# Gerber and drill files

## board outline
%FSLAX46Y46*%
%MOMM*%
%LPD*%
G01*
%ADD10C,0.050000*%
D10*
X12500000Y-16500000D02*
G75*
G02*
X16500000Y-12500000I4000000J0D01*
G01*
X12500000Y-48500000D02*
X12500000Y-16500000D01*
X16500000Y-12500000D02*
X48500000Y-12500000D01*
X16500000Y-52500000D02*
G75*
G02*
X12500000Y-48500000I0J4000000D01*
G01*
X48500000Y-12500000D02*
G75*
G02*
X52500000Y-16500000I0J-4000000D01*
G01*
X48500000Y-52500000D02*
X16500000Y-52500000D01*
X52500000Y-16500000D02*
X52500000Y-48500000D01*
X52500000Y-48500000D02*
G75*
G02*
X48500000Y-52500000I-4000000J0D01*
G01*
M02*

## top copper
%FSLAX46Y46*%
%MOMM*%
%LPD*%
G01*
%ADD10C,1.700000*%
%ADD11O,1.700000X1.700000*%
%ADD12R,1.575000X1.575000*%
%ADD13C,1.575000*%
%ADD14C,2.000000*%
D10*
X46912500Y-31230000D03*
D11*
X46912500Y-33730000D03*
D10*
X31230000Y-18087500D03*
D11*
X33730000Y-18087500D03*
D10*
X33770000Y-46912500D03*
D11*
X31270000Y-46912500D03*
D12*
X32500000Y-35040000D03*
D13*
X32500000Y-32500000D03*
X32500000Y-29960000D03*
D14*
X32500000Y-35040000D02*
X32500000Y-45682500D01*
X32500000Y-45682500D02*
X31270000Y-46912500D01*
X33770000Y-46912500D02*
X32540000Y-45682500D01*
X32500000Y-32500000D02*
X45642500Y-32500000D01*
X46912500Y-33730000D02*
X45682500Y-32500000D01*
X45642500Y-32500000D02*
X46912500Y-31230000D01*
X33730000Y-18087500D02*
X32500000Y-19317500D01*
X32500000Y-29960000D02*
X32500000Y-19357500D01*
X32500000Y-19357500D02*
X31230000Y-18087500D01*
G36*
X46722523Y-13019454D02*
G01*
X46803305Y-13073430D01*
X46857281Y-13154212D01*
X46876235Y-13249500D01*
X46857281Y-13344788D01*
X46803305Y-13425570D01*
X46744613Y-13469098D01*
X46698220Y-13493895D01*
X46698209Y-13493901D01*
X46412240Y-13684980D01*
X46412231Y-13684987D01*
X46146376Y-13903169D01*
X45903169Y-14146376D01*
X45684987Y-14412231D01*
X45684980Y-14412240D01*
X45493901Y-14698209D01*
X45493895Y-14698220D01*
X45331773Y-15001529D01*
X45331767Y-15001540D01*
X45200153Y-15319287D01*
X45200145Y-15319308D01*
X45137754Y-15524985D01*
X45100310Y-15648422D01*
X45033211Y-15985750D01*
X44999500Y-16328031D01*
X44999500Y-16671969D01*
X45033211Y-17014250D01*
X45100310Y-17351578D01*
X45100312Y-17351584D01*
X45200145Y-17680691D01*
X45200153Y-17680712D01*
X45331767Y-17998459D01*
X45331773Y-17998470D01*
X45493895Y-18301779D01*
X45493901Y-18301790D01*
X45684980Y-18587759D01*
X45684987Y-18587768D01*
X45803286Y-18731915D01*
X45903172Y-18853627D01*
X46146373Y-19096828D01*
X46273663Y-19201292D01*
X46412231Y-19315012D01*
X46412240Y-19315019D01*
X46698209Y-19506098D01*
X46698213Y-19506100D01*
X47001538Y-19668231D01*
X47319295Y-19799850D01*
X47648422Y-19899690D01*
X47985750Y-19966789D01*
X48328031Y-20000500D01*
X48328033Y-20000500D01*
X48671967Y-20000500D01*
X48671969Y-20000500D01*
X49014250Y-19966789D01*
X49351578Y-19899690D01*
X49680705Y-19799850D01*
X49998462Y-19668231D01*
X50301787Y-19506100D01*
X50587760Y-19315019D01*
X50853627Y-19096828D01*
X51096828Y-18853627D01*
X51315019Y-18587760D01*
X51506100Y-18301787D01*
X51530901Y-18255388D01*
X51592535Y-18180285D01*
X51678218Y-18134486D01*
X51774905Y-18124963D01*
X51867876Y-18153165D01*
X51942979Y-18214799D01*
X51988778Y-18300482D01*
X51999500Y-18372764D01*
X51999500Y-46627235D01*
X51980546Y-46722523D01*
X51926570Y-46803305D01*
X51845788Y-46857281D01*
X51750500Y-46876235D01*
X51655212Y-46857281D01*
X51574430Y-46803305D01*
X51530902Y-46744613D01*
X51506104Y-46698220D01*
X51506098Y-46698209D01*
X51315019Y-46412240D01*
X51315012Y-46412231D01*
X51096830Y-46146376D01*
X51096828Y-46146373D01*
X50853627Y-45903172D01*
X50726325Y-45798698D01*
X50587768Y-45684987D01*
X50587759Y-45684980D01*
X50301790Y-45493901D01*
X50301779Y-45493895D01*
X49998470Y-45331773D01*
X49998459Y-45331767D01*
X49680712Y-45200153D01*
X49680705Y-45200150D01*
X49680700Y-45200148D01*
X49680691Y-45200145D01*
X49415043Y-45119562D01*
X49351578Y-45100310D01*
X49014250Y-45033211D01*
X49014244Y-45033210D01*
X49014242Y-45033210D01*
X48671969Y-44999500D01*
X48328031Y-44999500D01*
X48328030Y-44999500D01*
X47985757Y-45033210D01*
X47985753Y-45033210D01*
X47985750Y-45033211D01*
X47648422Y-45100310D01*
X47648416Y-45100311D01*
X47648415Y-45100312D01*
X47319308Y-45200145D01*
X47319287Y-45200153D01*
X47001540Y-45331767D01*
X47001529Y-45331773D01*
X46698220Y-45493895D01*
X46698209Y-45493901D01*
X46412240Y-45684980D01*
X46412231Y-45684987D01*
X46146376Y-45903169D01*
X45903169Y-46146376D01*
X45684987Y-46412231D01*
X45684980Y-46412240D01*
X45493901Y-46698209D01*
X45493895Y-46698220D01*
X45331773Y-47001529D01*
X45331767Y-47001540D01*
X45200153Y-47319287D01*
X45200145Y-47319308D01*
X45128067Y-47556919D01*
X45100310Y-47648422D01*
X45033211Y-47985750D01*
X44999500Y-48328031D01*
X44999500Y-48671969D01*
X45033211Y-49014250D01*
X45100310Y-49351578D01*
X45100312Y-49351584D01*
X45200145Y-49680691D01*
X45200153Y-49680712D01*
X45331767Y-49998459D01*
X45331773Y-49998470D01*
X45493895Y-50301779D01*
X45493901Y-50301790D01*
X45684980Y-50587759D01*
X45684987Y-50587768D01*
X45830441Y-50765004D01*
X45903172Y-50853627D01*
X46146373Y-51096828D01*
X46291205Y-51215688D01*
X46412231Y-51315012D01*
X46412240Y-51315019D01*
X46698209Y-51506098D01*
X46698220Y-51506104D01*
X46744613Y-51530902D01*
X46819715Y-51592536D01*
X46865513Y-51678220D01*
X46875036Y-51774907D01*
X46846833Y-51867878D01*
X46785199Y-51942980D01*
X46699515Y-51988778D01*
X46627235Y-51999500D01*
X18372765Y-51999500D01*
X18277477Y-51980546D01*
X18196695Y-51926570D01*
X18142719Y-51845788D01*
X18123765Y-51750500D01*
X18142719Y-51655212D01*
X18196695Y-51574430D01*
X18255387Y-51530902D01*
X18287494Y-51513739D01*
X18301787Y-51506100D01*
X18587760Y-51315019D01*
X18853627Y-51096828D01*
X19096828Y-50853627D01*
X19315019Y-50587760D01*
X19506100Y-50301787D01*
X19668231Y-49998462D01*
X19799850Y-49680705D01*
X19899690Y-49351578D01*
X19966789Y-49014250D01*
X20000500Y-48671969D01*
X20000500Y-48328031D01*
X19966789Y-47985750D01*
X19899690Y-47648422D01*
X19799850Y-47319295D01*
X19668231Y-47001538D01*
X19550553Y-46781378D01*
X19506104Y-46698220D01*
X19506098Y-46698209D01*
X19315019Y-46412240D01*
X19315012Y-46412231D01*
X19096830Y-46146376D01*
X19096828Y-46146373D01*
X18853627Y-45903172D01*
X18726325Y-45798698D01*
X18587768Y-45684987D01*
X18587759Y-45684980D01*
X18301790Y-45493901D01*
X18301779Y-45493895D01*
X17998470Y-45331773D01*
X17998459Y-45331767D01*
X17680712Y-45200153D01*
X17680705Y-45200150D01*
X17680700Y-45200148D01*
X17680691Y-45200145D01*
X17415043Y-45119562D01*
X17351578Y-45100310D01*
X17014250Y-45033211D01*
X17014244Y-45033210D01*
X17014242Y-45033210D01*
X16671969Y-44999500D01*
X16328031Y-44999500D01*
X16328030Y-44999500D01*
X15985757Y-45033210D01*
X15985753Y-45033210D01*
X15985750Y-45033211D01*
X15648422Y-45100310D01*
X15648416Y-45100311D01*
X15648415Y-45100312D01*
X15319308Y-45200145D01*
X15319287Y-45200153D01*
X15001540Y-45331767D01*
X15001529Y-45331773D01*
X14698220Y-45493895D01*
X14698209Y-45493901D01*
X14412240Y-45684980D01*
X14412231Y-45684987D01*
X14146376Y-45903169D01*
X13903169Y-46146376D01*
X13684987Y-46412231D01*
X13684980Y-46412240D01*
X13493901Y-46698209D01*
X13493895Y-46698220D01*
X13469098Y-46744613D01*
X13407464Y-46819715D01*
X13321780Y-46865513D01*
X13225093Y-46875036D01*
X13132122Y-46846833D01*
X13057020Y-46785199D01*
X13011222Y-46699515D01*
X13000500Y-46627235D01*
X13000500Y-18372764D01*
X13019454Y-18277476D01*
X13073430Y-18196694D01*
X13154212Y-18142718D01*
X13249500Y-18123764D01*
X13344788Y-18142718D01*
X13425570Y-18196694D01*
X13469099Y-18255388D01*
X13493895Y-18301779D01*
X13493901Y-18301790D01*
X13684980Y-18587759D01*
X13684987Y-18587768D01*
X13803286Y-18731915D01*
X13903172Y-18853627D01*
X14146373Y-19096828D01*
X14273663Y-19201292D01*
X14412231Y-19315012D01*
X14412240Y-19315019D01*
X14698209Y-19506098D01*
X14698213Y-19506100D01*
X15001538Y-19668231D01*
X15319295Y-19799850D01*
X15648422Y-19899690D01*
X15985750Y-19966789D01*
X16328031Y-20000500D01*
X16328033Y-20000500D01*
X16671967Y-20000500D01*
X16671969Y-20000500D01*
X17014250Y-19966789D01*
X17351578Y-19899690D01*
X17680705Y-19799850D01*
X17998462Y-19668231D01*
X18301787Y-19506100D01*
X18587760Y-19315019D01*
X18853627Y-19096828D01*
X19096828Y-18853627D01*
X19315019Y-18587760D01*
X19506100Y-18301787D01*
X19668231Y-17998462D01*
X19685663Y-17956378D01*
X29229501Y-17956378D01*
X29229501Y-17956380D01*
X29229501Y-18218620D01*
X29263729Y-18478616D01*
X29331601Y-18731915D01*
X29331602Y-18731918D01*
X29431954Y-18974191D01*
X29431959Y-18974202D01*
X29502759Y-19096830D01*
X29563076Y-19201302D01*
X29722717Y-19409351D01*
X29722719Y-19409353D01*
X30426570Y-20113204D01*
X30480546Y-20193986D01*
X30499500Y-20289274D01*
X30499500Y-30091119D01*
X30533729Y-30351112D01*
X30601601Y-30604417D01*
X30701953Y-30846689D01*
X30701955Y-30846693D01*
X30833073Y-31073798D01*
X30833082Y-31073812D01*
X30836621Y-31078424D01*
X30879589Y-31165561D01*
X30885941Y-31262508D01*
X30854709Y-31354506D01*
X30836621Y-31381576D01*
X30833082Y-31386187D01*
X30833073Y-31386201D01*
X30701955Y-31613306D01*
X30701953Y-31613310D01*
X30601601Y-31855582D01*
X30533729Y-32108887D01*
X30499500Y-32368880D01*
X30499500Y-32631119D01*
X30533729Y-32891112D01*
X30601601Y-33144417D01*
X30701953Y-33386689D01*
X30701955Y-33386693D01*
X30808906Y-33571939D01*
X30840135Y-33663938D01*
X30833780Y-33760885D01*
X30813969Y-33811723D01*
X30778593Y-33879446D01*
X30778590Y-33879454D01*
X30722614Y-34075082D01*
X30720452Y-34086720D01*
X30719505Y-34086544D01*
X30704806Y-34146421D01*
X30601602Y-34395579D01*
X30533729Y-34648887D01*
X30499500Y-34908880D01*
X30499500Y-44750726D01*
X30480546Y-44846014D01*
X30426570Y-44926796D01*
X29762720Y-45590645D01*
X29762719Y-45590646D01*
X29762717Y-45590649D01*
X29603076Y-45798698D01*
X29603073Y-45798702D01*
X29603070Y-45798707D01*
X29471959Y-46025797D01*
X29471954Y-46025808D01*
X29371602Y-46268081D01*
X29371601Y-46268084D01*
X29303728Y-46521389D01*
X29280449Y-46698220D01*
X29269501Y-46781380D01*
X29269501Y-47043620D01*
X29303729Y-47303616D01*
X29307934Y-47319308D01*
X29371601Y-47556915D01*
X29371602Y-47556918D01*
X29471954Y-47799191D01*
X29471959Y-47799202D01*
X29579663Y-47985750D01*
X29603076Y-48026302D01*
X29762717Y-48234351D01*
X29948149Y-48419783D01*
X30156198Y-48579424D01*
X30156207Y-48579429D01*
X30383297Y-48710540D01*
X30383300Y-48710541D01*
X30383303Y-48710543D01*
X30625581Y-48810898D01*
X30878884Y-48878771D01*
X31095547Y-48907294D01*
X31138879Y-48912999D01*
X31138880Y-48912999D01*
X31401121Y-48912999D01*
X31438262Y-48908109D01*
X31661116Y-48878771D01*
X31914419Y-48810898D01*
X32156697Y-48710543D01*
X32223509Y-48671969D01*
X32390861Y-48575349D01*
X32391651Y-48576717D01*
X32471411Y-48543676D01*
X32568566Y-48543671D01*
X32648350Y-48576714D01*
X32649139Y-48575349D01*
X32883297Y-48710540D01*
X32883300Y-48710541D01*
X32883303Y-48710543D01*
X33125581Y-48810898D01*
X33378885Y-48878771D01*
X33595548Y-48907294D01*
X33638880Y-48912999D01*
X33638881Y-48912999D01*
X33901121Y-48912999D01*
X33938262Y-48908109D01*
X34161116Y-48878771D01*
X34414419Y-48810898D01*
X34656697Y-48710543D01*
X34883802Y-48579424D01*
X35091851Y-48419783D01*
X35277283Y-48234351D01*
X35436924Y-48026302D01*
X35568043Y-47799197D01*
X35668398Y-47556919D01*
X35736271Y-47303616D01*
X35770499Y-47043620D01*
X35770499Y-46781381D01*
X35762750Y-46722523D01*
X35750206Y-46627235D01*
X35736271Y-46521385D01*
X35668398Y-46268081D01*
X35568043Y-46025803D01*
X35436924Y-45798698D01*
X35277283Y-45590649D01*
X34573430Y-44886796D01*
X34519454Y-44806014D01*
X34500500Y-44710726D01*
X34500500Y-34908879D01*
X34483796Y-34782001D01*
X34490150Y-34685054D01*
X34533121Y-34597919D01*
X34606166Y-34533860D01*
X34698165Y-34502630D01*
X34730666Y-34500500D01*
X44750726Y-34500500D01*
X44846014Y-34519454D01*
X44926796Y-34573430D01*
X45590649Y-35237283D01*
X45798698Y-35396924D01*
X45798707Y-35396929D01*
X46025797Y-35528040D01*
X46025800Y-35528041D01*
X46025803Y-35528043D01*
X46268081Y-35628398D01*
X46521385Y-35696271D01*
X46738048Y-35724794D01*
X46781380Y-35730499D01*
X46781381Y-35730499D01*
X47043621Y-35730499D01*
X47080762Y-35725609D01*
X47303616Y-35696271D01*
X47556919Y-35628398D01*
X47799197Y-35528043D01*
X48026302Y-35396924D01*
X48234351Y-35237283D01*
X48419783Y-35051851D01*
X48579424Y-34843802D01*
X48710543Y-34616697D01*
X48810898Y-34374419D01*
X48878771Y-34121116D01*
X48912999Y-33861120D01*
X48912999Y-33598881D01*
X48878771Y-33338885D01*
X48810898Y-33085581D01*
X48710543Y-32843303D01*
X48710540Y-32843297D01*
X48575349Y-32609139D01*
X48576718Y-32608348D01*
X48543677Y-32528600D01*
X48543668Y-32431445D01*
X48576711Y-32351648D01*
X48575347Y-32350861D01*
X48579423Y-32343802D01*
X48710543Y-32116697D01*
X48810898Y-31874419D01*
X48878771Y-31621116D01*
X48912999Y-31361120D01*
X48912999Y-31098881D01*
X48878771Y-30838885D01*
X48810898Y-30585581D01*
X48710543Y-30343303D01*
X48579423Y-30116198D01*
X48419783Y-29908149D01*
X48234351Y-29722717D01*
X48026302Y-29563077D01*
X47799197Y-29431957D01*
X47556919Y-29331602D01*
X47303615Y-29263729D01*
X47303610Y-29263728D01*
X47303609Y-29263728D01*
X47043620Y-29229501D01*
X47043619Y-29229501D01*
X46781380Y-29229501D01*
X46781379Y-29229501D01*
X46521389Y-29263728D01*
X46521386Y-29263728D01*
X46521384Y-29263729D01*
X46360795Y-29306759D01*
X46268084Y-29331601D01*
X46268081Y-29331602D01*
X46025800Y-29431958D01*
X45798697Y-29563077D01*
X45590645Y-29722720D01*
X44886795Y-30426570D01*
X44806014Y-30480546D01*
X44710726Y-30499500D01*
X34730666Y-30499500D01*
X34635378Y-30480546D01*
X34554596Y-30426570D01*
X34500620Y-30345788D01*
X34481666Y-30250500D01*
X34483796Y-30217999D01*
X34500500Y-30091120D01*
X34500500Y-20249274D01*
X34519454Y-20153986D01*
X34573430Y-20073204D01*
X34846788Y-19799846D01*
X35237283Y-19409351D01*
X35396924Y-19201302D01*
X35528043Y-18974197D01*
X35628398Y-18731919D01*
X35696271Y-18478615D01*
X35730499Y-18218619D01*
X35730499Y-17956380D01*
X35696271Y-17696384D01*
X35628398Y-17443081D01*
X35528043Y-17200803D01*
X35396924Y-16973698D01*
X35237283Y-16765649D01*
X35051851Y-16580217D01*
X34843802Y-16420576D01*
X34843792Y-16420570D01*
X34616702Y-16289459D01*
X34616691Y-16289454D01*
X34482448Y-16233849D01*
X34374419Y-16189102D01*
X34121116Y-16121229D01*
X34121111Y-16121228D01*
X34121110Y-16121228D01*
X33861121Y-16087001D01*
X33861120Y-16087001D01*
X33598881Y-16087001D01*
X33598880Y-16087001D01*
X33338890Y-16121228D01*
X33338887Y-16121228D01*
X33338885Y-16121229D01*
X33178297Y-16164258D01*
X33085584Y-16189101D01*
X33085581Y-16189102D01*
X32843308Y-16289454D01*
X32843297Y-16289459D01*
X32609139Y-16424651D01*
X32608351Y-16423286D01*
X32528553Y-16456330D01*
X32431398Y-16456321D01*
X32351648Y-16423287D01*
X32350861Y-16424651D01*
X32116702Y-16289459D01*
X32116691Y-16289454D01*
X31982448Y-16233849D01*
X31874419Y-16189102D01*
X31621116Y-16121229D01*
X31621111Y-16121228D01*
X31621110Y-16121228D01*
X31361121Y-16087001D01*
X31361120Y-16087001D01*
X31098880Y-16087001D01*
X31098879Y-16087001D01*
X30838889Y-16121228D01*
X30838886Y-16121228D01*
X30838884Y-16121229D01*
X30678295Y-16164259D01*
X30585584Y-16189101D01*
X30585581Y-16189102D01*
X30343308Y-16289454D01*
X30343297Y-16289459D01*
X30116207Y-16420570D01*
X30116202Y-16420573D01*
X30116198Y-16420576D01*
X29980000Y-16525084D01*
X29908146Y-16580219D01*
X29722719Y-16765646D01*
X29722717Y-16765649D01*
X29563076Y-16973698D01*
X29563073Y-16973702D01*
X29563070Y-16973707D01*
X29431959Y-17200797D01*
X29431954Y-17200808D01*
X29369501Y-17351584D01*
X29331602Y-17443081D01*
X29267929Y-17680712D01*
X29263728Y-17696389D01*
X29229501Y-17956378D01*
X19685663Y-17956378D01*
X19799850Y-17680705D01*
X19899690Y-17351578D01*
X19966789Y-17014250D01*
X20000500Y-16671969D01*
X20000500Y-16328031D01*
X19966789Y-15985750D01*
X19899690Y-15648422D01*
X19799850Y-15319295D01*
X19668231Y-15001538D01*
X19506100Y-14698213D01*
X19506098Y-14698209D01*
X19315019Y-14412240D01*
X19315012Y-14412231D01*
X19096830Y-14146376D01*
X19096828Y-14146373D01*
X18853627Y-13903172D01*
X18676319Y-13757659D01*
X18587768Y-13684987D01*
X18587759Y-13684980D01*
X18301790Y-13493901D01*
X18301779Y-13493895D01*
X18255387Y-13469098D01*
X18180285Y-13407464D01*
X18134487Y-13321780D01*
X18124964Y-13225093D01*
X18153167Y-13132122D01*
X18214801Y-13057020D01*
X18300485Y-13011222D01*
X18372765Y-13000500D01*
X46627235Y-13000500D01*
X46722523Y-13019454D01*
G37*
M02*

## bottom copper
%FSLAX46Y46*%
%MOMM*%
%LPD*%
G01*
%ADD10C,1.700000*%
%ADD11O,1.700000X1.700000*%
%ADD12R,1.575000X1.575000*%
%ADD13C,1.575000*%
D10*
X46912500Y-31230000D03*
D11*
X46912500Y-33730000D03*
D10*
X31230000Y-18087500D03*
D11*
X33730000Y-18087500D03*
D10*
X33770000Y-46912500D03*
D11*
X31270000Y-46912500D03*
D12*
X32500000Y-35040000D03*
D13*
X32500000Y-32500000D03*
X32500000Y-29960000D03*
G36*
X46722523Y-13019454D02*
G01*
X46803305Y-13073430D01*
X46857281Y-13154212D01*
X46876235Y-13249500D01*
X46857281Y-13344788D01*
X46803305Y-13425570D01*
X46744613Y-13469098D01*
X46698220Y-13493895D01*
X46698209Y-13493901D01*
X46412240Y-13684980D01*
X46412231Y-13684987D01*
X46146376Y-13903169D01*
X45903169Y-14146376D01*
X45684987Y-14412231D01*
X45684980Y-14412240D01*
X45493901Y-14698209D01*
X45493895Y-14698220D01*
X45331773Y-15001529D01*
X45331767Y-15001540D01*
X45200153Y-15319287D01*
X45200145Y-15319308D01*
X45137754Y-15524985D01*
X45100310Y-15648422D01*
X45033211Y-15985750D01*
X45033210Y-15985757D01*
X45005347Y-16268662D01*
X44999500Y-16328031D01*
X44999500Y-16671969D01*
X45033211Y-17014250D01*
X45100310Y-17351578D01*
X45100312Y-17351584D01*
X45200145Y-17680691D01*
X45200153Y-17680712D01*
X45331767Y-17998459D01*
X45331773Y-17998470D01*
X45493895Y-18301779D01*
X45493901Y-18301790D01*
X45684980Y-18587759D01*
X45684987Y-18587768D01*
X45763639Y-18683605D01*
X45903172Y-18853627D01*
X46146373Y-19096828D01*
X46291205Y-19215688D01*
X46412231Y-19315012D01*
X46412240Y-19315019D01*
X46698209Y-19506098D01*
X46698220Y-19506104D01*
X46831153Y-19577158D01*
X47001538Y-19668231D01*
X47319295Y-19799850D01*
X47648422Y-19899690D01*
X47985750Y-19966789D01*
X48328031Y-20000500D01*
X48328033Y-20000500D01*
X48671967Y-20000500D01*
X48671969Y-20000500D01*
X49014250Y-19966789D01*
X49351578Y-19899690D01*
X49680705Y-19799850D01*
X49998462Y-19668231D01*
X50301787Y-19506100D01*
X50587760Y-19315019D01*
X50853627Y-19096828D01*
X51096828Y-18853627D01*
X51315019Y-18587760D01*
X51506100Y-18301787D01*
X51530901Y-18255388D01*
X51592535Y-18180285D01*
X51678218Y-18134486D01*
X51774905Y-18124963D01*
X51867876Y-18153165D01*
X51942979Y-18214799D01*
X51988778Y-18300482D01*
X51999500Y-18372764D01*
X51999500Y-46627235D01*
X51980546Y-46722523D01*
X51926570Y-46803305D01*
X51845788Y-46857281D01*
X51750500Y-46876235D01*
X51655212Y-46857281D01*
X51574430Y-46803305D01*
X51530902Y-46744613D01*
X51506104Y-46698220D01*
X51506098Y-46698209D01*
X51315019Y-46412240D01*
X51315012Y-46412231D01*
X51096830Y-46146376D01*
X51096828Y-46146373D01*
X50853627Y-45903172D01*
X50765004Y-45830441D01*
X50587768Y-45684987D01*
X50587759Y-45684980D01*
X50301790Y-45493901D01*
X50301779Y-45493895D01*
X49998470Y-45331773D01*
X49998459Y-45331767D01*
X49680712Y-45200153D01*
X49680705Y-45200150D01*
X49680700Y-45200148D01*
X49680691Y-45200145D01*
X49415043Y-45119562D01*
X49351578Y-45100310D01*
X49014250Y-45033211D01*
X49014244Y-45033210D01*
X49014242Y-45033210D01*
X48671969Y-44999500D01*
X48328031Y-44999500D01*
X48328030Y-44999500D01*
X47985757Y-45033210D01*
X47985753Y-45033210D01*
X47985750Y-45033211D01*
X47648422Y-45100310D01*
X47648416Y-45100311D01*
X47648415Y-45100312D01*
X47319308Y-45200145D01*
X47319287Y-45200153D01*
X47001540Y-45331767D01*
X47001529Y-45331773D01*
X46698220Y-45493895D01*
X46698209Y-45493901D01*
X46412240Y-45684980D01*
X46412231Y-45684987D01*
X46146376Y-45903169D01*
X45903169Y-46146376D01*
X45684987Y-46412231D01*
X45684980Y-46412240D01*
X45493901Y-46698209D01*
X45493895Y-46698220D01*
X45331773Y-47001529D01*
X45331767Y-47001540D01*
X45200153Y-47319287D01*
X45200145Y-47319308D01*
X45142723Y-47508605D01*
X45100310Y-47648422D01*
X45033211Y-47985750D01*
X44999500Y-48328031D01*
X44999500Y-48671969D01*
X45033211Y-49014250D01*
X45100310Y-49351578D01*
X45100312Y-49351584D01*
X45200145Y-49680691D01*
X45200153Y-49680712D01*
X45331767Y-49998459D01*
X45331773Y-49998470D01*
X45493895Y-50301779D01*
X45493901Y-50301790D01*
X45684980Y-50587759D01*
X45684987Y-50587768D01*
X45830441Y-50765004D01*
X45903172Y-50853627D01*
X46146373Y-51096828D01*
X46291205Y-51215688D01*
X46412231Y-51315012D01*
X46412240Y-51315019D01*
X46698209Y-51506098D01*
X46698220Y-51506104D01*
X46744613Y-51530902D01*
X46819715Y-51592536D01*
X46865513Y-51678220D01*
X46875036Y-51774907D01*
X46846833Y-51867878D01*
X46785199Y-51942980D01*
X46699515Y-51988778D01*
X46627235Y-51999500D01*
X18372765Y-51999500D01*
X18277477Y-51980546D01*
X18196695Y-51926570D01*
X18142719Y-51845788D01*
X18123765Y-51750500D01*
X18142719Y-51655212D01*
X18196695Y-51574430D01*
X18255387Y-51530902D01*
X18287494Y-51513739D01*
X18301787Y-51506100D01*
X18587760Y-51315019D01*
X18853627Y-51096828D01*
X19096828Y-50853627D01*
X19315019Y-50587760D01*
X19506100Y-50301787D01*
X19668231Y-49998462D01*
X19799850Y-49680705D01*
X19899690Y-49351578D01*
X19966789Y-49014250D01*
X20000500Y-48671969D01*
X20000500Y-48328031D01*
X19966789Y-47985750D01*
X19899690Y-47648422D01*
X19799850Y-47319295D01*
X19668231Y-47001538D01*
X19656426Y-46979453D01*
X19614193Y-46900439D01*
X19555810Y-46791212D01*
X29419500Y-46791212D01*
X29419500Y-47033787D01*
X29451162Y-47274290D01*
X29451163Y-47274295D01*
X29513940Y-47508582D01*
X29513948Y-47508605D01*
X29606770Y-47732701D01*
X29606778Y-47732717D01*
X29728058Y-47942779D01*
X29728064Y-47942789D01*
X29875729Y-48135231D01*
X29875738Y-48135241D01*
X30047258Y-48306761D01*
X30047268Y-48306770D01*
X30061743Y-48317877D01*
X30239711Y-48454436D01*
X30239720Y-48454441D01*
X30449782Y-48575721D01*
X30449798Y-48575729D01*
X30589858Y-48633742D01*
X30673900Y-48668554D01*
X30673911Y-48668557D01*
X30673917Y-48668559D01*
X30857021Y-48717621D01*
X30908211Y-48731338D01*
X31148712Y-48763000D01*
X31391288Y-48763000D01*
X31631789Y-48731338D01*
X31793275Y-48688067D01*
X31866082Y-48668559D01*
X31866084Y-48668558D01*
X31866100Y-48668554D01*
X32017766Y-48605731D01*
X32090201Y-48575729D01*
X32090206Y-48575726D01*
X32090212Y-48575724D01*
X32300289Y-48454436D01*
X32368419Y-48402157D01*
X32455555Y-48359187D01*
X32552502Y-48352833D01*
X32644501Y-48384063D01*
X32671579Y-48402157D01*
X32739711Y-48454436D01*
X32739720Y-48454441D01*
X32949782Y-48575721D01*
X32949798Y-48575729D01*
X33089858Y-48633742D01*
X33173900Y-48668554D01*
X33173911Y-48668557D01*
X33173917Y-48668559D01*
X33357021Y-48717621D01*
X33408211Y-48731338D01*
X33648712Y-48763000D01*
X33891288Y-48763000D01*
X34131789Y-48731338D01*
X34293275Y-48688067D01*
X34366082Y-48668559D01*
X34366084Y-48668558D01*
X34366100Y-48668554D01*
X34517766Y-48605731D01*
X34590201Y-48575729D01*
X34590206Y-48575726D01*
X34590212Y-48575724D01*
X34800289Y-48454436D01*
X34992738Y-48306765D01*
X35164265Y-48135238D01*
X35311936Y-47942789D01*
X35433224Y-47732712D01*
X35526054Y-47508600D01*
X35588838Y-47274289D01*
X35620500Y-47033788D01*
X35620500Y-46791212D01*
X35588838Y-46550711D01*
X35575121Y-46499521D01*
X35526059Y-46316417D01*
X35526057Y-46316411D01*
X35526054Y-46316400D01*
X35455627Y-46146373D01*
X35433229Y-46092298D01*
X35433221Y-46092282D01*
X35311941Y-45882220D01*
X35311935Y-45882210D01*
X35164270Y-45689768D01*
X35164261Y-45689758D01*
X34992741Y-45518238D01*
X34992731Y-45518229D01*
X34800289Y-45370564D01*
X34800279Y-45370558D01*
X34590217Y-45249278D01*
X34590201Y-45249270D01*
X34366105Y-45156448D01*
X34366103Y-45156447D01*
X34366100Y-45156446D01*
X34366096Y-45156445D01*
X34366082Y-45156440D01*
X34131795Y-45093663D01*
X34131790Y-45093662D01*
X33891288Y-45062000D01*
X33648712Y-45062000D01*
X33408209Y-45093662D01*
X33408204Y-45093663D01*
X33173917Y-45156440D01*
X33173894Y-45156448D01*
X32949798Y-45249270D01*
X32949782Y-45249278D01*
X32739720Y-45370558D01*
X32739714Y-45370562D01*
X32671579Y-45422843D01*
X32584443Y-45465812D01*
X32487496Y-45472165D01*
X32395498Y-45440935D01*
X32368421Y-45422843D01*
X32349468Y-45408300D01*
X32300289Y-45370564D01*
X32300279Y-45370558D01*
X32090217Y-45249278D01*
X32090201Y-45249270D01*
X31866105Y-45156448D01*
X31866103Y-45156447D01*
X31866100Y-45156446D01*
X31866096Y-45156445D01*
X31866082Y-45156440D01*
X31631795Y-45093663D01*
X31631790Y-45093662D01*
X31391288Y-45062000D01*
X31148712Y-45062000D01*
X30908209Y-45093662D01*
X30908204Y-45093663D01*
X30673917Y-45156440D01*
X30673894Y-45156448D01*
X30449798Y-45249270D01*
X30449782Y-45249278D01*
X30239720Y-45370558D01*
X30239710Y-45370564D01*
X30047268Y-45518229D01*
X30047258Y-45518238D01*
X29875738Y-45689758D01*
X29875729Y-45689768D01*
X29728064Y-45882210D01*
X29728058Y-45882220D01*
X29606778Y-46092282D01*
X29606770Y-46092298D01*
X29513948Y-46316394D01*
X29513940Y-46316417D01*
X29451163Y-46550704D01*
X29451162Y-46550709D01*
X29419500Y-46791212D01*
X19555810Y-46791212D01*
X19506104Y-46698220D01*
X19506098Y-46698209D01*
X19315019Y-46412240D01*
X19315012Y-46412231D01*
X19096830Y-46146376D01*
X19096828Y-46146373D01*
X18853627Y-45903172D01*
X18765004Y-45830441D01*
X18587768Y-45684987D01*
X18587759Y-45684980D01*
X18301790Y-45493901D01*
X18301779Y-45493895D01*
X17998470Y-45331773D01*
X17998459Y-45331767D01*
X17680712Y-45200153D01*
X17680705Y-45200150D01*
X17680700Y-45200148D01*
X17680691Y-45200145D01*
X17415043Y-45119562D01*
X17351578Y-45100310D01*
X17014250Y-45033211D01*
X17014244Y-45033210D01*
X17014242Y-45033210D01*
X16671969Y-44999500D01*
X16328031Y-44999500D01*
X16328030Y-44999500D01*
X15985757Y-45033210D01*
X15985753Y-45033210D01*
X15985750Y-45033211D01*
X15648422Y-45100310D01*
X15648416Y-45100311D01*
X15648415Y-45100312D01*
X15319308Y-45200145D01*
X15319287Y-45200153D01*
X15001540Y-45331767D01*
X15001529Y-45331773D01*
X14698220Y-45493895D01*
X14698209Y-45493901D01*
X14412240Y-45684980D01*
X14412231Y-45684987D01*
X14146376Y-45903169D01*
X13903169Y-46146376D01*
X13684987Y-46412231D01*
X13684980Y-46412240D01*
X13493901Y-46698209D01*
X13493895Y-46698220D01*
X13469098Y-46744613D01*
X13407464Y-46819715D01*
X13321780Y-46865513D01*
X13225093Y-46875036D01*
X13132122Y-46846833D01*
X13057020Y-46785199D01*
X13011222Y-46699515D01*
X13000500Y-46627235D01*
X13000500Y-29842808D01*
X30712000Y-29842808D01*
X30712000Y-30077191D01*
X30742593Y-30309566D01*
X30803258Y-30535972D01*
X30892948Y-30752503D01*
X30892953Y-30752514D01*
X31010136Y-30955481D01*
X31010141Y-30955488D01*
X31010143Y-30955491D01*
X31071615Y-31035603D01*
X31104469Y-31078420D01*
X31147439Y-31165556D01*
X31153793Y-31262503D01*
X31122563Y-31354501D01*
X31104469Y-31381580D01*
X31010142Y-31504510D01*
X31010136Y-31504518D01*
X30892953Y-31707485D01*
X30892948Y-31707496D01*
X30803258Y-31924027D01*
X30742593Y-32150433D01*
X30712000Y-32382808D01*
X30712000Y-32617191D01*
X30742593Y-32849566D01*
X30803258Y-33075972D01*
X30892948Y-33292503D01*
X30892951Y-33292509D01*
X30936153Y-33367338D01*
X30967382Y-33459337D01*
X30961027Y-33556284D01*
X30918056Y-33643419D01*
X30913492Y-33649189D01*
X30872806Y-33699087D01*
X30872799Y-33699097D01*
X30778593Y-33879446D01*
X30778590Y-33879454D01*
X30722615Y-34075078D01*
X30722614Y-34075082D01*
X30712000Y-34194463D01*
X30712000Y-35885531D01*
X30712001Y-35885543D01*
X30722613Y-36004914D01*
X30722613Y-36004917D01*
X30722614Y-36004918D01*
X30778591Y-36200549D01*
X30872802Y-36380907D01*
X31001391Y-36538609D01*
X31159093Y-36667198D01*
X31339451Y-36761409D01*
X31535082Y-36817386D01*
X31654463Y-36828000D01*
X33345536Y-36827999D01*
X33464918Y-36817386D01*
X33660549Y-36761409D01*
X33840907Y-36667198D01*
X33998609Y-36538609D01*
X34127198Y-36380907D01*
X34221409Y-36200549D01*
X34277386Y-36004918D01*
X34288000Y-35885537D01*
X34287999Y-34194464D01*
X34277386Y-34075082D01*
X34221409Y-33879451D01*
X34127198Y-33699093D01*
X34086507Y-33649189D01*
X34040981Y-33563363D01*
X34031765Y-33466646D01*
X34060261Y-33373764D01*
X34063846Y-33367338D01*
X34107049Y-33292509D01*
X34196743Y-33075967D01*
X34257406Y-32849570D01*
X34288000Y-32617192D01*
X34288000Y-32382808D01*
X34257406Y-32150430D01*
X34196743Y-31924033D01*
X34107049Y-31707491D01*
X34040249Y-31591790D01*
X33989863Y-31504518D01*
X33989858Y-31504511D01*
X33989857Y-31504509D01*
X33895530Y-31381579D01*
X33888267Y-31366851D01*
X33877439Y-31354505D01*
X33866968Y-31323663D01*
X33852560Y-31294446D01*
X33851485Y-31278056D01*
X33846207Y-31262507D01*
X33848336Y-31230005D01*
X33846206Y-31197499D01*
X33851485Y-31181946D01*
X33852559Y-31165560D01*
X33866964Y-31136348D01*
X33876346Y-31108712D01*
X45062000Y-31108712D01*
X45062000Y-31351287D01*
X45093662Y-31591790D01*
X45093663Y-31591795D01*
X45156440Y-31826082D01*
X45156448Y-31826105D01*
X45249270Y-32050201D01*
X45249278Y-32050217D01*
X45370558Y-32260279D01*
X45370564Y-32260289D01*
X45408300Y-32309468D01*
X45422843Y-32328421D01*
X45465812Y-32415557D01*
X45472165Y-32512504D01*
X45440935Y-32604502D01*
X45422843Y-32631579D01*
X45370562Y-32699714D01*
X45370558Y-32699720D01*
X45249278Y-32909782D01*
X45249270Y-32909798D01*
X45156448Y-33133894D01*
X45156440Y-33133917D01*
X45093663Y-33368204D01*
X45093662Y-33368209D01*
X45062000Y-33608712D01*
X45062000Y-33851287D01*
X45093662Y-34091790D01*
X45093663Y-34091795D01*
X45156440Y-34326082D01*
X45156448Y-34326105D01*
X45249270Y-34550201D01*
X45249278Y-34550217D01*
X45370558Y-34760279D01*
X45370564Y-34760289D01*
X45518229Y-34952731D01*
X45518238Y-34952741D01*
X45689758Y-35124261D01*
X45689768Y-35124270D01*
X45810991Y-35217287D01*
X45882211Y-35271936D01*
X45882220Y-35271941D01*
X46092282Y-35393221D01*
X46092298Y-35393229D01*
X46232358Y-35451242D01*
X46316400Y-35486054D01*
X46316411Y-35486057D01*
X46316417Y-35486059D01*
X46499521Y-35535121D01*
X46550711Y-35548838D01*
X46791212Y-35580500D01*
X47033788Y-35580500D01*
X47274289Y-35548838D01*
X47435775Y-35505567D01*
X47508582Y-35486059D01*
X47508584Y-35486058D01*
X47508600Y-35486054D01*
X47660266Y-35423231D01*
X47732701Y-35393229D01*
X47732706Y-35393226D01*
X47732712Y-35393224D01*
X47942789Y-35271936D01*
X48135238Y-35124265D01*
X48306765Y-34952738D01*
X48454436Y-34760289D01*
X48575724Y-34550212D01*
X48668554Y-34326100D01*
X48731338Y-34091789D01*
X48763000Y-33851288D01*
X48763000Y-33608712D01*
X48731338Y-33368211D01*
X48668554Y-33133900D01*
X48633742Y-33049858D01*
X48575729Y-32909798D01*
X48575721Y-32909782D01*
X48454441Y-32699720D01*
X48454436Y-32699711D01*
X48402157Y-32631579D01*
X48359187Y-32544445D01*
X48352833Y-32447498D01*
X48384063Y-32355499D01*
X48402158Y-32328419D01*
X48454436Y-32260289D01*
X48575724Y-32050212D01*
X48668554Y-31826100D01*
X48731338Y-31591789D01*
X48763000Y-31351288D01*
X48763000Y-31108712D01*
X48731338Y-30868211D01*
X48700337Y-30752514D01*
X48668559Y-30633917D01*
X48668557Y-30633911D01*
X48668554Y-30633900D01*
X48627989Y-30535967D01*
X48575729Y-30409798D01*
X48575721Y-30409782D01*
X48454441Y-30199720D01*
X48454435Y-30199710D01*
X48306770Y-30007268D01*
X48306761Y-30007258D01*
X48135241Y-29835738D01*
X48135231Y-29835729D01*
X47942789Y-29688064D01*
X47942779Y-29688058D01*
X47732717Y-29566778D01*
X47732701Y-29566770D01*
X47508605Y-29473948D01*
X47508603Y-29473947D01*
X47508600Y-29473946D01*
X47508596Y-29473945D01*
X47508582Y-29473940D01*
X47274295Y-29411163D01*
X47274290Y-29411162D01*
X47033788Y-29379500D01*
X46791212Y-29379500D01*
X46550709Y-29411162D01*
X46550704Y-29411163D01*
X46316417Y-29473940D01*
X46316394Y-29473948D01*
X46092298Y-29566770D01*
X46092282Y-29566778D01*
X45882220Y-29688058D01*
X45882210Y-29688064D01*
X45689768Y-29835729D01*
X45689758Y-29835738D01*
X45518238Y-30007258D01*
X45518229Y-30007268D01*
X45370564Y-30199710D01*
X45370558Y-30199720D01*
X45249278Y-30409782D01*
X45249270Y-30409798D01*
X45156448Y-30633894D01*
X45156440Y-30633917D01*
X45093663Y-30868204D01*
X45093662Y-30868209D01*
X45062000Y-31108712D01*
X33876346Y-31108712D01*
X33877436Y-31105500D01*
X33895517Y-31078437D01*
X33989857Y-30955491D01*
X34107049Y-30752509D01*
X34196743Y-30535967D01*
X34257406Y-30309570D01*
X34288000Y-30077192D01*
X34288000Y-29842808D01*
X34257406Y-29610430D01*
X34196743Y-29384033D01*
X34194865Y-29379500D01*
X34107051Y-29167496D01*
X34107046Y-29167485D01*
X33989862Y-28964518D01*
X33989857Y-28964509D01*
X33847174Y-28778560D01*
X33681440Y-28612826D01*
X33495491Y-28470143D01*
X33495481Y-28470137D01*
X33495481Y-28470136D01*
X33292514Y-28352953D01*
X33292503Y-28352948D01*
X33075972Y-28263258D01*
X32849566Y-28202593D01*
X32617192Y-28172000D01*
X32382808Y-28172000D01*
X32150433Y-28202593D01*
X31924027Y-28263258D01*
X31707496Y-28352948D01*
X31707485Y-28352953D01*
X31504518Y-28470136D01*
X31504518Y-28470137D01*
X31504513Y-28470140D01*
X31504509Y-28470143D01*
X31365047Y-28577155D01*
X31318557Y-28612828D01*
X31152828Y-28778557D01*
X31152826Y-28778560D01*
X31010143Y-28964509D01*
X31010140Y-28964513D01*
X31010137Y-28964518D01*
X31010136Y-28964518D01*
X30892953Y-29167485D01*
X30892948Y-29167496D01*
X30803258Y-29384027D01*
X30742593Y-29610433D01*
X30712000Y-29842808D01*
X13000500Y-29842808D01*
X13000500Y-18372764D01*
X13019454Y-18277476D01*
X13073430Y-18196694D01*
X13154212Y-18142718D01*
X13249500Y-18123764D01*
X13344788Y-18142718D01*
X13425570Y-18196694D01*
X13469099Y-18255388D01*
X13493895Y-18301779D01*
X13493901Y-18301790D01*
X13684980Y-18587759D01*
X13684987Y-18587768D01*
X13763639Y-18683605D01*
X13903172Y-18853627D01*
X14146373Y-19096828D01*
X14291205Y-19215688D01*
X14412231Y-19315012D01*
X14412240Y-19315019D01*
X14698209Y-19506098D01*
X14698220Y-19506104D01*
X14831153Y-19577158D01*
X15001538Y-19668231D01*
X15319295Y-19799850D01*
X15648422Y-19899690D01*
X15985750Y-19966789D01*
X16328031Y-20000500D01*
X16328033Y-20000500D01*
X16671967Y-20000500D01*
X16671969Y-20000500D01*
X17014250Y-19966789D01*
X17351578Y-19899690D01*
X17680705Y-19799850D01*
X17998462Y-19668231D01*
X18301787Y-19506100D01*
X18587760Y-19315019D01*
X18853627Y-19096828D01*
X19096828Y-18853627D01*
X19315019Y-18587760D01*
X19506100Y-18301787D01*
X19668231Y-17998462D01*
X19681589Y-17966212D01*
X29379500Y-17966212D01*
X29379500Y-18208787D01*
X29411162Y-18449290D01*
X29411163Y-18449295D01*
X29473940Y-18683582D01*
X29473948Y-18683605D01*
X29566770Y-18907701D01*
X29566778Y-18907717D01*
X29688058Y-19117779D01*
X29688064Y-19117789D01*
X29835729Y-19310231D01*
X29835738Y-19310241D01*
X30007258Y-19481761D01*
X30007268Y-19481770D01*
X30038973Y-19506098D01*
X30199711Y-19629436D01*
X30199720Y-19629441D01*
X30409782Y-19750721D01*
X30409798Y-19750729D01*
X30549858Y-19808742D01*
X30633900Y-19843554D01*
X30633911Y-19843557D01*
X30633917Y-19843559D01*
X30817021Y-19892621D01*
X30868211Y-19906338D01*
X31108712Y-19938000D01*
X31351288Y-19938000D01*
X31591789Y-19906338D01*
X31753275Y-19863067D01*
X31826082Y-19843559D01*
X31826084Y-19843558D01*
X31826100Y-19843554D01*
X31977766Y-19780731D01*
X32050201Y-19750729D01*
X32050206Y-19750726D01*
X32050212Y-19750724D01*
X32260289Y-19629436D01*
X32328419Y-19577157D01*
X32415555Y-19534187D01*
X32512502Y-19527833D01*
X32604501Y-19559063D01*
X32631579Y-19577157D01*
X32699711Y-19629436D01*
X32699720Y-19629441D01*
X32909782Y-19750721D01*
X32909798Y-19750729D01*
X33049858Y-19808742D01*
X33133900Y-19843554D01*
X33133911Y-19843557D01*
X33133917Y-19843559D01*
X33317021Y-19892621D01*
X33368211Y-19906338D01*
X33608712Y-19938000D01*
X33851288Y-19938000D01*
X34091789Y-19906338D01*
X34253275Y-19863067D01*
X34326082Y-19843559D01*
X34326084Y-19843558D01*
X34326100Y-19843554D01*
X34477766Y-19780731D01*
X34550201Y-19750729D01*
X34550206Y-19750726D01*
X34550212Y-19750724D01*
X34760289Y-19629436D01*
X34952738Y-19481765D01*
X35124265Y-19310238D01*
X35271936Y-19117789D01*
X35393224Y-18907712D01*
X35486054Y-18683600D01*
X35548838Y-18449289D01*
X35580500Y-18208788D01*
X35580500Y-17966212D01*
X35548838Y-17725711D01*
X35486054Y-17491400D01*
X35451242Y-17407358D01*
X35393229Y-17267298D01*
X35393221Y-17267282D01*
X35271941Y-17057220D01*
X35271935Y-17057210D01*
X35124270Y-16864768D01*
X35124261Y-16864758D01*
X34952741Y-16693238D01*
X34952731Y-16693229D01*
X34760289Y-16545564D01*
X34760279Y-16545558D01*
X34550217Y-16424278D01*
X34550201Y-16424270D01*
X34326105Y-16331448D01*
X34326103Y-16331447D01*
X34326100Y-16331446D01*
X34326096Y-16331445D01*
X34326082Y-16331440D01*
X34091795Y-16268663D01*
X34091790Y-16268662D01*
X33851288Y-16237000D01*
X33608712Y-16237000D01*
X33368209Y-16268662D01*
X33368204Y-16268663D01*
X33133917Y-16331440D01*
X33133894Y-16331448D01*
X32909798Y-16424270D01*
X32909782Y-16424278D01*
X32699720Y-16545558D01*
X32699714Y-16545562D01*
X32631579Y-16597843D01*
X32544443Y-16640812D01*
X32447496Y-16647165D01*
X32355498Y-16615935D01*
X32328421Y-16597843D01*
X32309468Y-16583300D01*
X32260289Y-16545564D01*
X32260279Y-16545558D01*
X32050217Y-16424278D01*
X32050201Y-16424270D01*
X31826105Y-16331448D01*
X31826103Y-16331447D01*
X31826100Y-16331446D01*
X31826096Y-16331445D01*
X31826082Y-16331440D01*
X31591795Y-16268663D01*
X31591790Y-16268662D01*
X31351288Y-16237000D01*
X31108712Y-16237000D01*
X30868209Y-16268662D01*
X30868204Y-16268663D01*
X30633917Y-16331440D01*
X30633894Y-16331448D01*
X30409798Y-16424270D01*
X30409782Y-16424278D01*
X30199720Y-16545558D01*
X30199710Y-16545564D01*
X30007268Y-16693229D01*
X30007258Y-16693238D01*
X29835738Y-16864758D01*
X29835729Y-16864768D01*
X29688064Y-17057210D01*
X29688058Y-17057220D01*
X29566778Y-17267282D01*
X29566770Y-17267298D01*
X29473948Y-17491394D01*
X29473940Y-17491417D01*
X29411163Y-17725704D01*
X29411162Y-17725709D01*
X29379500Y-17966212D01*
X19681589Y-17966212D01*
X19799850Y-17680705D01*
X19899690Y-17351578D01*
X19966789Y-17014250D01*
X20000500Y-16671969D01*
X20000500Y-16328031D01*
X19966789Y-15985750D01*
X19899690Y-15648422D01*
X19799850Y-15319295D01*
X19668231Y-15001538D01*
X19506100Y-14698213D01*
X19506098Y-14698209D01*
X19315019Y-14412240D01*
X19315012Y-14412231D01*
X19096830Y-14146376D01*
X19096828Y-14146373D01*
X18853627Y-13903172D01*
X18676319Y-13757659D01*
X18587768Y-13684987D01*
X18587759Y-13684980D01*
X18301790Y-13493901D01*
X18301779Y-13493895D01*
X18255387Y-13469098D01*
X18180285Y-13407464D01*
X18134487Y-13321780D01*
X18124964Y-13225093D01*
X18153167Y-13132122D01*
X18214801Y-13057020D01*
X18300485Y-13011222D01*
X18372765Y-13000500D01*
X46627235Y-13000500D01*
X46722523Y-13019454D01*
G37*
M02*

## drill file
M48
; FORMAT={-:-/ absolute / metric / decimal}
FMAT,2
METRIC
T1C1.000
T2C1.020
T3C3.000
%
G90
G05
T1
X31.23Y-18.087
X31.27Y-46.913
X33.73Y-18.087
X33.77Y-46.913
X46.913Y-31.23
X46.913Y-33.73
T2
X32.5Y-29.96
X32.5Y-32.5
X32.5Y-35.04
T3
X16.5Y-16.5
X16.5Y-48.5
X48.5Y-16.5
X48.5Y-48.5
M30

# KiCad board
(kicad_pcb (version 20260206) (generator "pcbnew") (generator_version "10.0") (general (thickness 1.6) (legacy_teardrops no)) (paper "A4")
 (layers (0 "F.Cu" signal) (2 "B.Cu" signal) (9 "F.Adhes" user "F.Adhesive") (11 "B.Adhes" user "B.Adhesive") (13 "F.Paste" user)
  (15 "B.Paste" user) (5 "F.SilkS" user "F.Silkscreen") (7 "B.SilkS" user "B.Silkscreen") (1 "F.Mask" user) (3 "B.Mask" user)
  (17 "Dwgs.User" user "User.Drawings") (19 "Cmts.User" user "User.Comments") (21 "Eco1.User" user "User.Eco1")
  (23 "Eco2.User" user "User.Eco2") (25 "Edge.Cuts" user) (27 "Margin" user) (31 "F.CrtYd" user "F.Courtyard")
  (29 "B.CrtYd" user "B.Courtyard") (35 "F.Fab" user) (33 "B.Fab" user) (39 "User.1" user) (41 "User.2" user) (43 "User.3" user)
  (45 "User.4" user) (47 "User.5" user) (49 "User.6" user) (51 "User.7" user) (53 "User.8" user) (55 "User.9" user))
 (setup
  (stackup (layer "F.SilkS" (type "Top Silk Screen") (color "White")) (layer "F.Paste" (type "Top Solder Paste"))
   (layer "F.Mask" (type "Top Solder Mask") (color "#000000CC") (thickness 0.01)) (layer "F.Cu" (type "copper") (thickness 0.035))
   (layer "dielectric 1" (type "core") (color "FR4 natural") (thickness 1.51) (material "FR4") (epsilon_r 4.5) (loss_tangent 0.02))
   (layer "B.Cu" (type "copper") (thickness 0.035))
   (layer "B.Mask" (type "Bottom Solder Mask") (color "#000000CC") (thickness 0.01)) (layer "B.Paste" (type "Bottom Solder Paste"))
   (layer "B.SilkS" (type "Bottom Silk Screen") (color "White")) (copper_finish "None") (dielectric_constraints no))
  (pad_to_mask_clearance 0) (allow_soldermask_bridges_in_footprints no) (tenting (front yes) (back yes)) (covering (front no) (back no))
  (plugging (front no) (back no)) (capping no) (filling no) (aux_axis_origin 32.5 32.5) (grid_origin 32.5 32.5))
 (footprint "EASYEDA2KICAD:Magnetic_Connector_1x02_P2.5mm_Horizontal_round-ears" (layer "F.Cu") (at 47.0125 32.5)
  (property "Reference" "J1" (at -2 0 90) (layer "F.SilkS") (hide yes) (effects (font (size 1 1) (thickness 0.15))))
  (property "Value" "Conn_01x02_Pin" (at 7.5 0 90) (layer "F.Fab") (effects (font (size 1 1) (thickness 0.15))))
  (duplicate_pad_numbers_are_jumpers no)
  (pad "1" thru_hole circle (at -0.1 -1.27) (size 1.7 1.7) (drill 1) (layers "*.Cu" "*.Mask") (remove_unused_layers no)
   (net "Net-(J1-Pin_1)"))
  (pad "2" thru_hole oval (at -0.1 1.23) (size 1.7 1.7) (drill 1) (layers "*.Cu" "*.Mask") (remove_unused_layers no) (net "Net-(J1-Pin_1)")))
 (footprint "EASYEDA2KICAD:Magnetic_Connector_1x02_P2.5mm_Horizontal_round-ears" (layer "F.Cu") (at 32.5 17.9875 90)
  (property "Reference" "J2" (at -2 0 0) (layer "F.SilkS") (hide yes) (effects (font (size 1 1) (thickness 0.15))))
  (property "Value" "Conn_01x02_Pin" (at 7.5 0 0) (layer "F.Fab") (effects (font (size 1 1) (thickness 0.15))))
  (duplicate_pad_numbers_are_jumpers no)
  (pad "1" thru_hole circle (at -0.1 -1.27 90) (size 1.7 1.7) (drill 1) (layers "*.Cu" "*.Mask") (remove_unused_layers no)
   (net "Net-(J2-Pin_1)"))
  (pad "2" thru_hole oval (at -0.1 1.23 90) (size 1.7 1.7) (drill 1) (layers "*.Cu" "*.Mask") (remove_unused_layers no)
   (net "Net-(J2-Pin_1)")))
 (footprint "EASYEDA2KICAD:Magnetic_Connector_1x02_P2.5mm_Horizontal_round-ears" (layer "F.Cu") (at 32.5 47.0125 -90)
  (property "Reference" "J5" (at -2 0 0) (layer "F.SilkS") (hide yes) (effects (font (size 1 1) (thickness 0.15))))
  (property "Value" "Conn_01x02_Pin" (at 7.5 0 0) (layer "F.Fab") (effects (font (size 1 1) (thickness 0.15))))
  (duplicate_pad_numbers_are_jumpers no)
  (pad "1" thru_hole circle (at -0.1 -1.27 270) (size 1.7 1.7) (drill 1) (layers "*.Cu" "*.Mask") (remove_unused_layers no) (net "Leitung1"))
  (pad "2" thru_hole oval (at -0.1 1.23 270) (size 1.7 1.7) (drill 1) (layers "*.Cu" "*.Mask") (remove_unused_layers no) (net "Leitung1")))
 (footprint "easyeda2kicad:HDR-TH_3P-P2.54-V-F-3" (layer "B.Cu") (at 32.5 32.5 90)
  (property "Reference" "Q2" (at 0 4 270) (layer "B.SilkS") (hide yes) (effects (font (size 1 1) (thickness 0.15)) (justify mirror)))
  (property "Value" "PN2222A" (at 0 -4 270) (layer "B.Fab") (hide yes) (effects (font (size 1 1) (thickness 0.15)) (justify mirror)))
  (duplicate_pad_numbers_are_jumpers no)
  (pad "1" thru_hole rect (at -2.54 0 90) (size 1.575 1.575) (drill 1.020014) (layers "*.Cu" "*.Mask") (remove_unused_layers no)
   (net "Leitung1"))
  (pad "2" thru_hole circle (at 0 0 90) (size 1.575 1.575) (drill 1.020014) (layers "*.Cu" "*.Mask") (remove_unused_layers no)
   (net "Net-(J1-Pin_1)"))
  (pad "3" thru_hole circle (at 2.54 0 90) (size 1.575 1.575) (drill 1.020014) (layers "*.Cu" "*.Mask") (remove_unused_layers no)
   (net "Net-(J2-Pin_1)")))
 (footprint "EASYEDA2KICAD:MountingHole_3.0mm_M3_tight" (layer "B.Cu") (at 16.5 16.5 180)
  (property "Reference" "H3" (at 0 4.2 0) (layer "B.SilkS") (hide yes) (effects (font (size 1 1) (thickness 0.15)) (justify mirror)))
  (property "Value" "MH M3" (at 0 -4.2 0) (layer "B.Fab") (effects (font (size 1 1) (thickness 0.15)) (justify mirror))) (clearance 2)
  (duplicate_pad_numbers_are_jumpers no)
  (pad "" np_thru_hole circle (at 0 0 180) (size 3 3) (drill 3) (layers "*.Cu" "*.Mask")))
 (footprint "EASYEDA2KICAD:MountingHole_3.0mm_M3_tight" (layer "B.Cu") (at 48.5 16.5 180)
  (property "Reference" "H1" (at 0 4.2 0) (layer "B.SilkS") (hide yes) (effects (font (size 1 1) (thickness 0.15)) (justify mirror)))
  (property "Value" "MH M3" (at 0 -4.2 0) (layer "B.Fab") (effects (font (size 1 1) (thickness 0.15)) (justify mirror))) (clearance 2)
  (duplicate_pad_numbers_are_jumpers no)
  (pad "" np_thru_hole circle (at 0 0 180) (size 3 3) (drill 3) (layers "*.Cu" "*.Mask")))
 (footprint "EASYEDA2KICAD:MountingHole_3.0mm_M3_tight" (layer "B.Cu") (at 16.5 48.5 180)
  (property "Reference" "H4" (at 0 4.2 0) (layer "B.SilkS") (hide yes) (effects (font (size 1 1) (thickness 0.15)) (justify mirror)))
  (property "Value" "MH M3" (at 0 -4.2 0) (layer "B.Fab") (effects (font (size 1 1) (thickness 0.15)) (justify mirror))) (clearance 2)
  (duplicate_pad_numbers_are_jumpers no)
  (pad "" np_thru_hole circle (at 0 0 180) (size 3 3) (drill 3) (layers "*.Cu" "*.Mask")))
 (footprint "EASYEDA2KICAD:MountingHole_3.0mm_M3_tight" (layer "B.Cu") (at 48.5 48.5 180)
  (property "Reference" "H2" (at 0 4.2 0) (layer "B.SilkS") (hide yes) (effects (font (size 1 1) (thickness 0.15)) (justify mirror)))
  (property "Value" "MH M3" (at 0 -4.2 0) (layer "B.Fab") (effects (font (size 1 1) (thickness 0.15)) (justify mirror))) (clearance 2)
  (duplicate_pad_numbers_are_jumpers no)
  (pad "" np_thru_hole circle (at 0 0 180) (size 3 3) (drill 3) (layers "*.Cu" "*.Mask")))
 (gr_arc (start 12.5 16.5) (mid 13.671573 13.671573) (end 16.5 12.5) (stroke (width 0.05) (type default)) (layer "Edge.Cuts"))
 (gr_line (start 12.5 48.5) (end 12.5 16.5) (stroke (width 0.05) (type default)) (layer "Edge.Cuts"))
 (gr_line (start 16.5 12.5) (end 48.5 12.5) (stroke (width 0.05) (type default)) (layer "Edge.Cuts"))
 (gr_arc (start 16.5 52.5) (mid 13.671573 51.328427) (end 12.5 48.5) (stroke (width 0.05) (type default)) (layer "Edge.Cuts"))
 (gr_arc (start 48.5 12.5) (mid 51.328427 13.671573) (end 52.5 16.5) (stroke (width 0.05) (type default)) (layer "Edge.Cuts"))
 (gr_line (start 48.5 52.5) (end 16.5 52.5) (stroke (width 0.05) (type default)) (layer "Edge.Cuts"))
 (gr_line (start 52.5 16.5) (end 52.5 48.5) (stroke (width 0.05) (type default)) (layer "Edge.Cuts"))
 (gr_arc (start 52.5 48.5) (mid 51.328427 51.328427) (end 48.5 52.5) (stroke (width 0.05) (type default)) (layer "Edge.Cuts"))
 (segment (start 32.5 35.04) (end 32.5 45.6825) (width 2) (layer "F.Cu") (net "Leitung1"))
 (segment (start 32.5 45.6825) (end 31.27 46.9125) (width 2) (layer "F.Cu") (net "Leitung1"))
 (segment (start 33.77 46.9125) (end 32.54 45.6825) (width 2) (layer "F.Cu") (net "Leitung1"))
 (segment (start 32.5 32.5) (end 45.6425 32.5) (width 2) (layer "F.Cu") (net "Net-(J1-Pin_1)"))
 (segment (start 46.9125 33.73) (end 45.6825 32.5) (width 2) (layer "F.Cu") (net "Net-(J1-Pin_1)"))
 (segment (start 45.6425 32.5) (end 46.9125 31.23) (width 2) (layer "F.Cu") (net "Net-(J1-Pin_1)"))
 (segment (start 33.73 18.0875) (end 32.5 19.3175) (width 2) (layer "F.Cu") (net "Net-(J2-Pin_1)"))
 (segment (start 32.5 29.96) (end 32.5 19.3575) (width 2) (layer "F.Cu") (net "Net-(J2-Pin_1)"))
 (segment (start 32.5 19.3575) (end 31.23 18.0875) (width 2) (layer "F.Cu") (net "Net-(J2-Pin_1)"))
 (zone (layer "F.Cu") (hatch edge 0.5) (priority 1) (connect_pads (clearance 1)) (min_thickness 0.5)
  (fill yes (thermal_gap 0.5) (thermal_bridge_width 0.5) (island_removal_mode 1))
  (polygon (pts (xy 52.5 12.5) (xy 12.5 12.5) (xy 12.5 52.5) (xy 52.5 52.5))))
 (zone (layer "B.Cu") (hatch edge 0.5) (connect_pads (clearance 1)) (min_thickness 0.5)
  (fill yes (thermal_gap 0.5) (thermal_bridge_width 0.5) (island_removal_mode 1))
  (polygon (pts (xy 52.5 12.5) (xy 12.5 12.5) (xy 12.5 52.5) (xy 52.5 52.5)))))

